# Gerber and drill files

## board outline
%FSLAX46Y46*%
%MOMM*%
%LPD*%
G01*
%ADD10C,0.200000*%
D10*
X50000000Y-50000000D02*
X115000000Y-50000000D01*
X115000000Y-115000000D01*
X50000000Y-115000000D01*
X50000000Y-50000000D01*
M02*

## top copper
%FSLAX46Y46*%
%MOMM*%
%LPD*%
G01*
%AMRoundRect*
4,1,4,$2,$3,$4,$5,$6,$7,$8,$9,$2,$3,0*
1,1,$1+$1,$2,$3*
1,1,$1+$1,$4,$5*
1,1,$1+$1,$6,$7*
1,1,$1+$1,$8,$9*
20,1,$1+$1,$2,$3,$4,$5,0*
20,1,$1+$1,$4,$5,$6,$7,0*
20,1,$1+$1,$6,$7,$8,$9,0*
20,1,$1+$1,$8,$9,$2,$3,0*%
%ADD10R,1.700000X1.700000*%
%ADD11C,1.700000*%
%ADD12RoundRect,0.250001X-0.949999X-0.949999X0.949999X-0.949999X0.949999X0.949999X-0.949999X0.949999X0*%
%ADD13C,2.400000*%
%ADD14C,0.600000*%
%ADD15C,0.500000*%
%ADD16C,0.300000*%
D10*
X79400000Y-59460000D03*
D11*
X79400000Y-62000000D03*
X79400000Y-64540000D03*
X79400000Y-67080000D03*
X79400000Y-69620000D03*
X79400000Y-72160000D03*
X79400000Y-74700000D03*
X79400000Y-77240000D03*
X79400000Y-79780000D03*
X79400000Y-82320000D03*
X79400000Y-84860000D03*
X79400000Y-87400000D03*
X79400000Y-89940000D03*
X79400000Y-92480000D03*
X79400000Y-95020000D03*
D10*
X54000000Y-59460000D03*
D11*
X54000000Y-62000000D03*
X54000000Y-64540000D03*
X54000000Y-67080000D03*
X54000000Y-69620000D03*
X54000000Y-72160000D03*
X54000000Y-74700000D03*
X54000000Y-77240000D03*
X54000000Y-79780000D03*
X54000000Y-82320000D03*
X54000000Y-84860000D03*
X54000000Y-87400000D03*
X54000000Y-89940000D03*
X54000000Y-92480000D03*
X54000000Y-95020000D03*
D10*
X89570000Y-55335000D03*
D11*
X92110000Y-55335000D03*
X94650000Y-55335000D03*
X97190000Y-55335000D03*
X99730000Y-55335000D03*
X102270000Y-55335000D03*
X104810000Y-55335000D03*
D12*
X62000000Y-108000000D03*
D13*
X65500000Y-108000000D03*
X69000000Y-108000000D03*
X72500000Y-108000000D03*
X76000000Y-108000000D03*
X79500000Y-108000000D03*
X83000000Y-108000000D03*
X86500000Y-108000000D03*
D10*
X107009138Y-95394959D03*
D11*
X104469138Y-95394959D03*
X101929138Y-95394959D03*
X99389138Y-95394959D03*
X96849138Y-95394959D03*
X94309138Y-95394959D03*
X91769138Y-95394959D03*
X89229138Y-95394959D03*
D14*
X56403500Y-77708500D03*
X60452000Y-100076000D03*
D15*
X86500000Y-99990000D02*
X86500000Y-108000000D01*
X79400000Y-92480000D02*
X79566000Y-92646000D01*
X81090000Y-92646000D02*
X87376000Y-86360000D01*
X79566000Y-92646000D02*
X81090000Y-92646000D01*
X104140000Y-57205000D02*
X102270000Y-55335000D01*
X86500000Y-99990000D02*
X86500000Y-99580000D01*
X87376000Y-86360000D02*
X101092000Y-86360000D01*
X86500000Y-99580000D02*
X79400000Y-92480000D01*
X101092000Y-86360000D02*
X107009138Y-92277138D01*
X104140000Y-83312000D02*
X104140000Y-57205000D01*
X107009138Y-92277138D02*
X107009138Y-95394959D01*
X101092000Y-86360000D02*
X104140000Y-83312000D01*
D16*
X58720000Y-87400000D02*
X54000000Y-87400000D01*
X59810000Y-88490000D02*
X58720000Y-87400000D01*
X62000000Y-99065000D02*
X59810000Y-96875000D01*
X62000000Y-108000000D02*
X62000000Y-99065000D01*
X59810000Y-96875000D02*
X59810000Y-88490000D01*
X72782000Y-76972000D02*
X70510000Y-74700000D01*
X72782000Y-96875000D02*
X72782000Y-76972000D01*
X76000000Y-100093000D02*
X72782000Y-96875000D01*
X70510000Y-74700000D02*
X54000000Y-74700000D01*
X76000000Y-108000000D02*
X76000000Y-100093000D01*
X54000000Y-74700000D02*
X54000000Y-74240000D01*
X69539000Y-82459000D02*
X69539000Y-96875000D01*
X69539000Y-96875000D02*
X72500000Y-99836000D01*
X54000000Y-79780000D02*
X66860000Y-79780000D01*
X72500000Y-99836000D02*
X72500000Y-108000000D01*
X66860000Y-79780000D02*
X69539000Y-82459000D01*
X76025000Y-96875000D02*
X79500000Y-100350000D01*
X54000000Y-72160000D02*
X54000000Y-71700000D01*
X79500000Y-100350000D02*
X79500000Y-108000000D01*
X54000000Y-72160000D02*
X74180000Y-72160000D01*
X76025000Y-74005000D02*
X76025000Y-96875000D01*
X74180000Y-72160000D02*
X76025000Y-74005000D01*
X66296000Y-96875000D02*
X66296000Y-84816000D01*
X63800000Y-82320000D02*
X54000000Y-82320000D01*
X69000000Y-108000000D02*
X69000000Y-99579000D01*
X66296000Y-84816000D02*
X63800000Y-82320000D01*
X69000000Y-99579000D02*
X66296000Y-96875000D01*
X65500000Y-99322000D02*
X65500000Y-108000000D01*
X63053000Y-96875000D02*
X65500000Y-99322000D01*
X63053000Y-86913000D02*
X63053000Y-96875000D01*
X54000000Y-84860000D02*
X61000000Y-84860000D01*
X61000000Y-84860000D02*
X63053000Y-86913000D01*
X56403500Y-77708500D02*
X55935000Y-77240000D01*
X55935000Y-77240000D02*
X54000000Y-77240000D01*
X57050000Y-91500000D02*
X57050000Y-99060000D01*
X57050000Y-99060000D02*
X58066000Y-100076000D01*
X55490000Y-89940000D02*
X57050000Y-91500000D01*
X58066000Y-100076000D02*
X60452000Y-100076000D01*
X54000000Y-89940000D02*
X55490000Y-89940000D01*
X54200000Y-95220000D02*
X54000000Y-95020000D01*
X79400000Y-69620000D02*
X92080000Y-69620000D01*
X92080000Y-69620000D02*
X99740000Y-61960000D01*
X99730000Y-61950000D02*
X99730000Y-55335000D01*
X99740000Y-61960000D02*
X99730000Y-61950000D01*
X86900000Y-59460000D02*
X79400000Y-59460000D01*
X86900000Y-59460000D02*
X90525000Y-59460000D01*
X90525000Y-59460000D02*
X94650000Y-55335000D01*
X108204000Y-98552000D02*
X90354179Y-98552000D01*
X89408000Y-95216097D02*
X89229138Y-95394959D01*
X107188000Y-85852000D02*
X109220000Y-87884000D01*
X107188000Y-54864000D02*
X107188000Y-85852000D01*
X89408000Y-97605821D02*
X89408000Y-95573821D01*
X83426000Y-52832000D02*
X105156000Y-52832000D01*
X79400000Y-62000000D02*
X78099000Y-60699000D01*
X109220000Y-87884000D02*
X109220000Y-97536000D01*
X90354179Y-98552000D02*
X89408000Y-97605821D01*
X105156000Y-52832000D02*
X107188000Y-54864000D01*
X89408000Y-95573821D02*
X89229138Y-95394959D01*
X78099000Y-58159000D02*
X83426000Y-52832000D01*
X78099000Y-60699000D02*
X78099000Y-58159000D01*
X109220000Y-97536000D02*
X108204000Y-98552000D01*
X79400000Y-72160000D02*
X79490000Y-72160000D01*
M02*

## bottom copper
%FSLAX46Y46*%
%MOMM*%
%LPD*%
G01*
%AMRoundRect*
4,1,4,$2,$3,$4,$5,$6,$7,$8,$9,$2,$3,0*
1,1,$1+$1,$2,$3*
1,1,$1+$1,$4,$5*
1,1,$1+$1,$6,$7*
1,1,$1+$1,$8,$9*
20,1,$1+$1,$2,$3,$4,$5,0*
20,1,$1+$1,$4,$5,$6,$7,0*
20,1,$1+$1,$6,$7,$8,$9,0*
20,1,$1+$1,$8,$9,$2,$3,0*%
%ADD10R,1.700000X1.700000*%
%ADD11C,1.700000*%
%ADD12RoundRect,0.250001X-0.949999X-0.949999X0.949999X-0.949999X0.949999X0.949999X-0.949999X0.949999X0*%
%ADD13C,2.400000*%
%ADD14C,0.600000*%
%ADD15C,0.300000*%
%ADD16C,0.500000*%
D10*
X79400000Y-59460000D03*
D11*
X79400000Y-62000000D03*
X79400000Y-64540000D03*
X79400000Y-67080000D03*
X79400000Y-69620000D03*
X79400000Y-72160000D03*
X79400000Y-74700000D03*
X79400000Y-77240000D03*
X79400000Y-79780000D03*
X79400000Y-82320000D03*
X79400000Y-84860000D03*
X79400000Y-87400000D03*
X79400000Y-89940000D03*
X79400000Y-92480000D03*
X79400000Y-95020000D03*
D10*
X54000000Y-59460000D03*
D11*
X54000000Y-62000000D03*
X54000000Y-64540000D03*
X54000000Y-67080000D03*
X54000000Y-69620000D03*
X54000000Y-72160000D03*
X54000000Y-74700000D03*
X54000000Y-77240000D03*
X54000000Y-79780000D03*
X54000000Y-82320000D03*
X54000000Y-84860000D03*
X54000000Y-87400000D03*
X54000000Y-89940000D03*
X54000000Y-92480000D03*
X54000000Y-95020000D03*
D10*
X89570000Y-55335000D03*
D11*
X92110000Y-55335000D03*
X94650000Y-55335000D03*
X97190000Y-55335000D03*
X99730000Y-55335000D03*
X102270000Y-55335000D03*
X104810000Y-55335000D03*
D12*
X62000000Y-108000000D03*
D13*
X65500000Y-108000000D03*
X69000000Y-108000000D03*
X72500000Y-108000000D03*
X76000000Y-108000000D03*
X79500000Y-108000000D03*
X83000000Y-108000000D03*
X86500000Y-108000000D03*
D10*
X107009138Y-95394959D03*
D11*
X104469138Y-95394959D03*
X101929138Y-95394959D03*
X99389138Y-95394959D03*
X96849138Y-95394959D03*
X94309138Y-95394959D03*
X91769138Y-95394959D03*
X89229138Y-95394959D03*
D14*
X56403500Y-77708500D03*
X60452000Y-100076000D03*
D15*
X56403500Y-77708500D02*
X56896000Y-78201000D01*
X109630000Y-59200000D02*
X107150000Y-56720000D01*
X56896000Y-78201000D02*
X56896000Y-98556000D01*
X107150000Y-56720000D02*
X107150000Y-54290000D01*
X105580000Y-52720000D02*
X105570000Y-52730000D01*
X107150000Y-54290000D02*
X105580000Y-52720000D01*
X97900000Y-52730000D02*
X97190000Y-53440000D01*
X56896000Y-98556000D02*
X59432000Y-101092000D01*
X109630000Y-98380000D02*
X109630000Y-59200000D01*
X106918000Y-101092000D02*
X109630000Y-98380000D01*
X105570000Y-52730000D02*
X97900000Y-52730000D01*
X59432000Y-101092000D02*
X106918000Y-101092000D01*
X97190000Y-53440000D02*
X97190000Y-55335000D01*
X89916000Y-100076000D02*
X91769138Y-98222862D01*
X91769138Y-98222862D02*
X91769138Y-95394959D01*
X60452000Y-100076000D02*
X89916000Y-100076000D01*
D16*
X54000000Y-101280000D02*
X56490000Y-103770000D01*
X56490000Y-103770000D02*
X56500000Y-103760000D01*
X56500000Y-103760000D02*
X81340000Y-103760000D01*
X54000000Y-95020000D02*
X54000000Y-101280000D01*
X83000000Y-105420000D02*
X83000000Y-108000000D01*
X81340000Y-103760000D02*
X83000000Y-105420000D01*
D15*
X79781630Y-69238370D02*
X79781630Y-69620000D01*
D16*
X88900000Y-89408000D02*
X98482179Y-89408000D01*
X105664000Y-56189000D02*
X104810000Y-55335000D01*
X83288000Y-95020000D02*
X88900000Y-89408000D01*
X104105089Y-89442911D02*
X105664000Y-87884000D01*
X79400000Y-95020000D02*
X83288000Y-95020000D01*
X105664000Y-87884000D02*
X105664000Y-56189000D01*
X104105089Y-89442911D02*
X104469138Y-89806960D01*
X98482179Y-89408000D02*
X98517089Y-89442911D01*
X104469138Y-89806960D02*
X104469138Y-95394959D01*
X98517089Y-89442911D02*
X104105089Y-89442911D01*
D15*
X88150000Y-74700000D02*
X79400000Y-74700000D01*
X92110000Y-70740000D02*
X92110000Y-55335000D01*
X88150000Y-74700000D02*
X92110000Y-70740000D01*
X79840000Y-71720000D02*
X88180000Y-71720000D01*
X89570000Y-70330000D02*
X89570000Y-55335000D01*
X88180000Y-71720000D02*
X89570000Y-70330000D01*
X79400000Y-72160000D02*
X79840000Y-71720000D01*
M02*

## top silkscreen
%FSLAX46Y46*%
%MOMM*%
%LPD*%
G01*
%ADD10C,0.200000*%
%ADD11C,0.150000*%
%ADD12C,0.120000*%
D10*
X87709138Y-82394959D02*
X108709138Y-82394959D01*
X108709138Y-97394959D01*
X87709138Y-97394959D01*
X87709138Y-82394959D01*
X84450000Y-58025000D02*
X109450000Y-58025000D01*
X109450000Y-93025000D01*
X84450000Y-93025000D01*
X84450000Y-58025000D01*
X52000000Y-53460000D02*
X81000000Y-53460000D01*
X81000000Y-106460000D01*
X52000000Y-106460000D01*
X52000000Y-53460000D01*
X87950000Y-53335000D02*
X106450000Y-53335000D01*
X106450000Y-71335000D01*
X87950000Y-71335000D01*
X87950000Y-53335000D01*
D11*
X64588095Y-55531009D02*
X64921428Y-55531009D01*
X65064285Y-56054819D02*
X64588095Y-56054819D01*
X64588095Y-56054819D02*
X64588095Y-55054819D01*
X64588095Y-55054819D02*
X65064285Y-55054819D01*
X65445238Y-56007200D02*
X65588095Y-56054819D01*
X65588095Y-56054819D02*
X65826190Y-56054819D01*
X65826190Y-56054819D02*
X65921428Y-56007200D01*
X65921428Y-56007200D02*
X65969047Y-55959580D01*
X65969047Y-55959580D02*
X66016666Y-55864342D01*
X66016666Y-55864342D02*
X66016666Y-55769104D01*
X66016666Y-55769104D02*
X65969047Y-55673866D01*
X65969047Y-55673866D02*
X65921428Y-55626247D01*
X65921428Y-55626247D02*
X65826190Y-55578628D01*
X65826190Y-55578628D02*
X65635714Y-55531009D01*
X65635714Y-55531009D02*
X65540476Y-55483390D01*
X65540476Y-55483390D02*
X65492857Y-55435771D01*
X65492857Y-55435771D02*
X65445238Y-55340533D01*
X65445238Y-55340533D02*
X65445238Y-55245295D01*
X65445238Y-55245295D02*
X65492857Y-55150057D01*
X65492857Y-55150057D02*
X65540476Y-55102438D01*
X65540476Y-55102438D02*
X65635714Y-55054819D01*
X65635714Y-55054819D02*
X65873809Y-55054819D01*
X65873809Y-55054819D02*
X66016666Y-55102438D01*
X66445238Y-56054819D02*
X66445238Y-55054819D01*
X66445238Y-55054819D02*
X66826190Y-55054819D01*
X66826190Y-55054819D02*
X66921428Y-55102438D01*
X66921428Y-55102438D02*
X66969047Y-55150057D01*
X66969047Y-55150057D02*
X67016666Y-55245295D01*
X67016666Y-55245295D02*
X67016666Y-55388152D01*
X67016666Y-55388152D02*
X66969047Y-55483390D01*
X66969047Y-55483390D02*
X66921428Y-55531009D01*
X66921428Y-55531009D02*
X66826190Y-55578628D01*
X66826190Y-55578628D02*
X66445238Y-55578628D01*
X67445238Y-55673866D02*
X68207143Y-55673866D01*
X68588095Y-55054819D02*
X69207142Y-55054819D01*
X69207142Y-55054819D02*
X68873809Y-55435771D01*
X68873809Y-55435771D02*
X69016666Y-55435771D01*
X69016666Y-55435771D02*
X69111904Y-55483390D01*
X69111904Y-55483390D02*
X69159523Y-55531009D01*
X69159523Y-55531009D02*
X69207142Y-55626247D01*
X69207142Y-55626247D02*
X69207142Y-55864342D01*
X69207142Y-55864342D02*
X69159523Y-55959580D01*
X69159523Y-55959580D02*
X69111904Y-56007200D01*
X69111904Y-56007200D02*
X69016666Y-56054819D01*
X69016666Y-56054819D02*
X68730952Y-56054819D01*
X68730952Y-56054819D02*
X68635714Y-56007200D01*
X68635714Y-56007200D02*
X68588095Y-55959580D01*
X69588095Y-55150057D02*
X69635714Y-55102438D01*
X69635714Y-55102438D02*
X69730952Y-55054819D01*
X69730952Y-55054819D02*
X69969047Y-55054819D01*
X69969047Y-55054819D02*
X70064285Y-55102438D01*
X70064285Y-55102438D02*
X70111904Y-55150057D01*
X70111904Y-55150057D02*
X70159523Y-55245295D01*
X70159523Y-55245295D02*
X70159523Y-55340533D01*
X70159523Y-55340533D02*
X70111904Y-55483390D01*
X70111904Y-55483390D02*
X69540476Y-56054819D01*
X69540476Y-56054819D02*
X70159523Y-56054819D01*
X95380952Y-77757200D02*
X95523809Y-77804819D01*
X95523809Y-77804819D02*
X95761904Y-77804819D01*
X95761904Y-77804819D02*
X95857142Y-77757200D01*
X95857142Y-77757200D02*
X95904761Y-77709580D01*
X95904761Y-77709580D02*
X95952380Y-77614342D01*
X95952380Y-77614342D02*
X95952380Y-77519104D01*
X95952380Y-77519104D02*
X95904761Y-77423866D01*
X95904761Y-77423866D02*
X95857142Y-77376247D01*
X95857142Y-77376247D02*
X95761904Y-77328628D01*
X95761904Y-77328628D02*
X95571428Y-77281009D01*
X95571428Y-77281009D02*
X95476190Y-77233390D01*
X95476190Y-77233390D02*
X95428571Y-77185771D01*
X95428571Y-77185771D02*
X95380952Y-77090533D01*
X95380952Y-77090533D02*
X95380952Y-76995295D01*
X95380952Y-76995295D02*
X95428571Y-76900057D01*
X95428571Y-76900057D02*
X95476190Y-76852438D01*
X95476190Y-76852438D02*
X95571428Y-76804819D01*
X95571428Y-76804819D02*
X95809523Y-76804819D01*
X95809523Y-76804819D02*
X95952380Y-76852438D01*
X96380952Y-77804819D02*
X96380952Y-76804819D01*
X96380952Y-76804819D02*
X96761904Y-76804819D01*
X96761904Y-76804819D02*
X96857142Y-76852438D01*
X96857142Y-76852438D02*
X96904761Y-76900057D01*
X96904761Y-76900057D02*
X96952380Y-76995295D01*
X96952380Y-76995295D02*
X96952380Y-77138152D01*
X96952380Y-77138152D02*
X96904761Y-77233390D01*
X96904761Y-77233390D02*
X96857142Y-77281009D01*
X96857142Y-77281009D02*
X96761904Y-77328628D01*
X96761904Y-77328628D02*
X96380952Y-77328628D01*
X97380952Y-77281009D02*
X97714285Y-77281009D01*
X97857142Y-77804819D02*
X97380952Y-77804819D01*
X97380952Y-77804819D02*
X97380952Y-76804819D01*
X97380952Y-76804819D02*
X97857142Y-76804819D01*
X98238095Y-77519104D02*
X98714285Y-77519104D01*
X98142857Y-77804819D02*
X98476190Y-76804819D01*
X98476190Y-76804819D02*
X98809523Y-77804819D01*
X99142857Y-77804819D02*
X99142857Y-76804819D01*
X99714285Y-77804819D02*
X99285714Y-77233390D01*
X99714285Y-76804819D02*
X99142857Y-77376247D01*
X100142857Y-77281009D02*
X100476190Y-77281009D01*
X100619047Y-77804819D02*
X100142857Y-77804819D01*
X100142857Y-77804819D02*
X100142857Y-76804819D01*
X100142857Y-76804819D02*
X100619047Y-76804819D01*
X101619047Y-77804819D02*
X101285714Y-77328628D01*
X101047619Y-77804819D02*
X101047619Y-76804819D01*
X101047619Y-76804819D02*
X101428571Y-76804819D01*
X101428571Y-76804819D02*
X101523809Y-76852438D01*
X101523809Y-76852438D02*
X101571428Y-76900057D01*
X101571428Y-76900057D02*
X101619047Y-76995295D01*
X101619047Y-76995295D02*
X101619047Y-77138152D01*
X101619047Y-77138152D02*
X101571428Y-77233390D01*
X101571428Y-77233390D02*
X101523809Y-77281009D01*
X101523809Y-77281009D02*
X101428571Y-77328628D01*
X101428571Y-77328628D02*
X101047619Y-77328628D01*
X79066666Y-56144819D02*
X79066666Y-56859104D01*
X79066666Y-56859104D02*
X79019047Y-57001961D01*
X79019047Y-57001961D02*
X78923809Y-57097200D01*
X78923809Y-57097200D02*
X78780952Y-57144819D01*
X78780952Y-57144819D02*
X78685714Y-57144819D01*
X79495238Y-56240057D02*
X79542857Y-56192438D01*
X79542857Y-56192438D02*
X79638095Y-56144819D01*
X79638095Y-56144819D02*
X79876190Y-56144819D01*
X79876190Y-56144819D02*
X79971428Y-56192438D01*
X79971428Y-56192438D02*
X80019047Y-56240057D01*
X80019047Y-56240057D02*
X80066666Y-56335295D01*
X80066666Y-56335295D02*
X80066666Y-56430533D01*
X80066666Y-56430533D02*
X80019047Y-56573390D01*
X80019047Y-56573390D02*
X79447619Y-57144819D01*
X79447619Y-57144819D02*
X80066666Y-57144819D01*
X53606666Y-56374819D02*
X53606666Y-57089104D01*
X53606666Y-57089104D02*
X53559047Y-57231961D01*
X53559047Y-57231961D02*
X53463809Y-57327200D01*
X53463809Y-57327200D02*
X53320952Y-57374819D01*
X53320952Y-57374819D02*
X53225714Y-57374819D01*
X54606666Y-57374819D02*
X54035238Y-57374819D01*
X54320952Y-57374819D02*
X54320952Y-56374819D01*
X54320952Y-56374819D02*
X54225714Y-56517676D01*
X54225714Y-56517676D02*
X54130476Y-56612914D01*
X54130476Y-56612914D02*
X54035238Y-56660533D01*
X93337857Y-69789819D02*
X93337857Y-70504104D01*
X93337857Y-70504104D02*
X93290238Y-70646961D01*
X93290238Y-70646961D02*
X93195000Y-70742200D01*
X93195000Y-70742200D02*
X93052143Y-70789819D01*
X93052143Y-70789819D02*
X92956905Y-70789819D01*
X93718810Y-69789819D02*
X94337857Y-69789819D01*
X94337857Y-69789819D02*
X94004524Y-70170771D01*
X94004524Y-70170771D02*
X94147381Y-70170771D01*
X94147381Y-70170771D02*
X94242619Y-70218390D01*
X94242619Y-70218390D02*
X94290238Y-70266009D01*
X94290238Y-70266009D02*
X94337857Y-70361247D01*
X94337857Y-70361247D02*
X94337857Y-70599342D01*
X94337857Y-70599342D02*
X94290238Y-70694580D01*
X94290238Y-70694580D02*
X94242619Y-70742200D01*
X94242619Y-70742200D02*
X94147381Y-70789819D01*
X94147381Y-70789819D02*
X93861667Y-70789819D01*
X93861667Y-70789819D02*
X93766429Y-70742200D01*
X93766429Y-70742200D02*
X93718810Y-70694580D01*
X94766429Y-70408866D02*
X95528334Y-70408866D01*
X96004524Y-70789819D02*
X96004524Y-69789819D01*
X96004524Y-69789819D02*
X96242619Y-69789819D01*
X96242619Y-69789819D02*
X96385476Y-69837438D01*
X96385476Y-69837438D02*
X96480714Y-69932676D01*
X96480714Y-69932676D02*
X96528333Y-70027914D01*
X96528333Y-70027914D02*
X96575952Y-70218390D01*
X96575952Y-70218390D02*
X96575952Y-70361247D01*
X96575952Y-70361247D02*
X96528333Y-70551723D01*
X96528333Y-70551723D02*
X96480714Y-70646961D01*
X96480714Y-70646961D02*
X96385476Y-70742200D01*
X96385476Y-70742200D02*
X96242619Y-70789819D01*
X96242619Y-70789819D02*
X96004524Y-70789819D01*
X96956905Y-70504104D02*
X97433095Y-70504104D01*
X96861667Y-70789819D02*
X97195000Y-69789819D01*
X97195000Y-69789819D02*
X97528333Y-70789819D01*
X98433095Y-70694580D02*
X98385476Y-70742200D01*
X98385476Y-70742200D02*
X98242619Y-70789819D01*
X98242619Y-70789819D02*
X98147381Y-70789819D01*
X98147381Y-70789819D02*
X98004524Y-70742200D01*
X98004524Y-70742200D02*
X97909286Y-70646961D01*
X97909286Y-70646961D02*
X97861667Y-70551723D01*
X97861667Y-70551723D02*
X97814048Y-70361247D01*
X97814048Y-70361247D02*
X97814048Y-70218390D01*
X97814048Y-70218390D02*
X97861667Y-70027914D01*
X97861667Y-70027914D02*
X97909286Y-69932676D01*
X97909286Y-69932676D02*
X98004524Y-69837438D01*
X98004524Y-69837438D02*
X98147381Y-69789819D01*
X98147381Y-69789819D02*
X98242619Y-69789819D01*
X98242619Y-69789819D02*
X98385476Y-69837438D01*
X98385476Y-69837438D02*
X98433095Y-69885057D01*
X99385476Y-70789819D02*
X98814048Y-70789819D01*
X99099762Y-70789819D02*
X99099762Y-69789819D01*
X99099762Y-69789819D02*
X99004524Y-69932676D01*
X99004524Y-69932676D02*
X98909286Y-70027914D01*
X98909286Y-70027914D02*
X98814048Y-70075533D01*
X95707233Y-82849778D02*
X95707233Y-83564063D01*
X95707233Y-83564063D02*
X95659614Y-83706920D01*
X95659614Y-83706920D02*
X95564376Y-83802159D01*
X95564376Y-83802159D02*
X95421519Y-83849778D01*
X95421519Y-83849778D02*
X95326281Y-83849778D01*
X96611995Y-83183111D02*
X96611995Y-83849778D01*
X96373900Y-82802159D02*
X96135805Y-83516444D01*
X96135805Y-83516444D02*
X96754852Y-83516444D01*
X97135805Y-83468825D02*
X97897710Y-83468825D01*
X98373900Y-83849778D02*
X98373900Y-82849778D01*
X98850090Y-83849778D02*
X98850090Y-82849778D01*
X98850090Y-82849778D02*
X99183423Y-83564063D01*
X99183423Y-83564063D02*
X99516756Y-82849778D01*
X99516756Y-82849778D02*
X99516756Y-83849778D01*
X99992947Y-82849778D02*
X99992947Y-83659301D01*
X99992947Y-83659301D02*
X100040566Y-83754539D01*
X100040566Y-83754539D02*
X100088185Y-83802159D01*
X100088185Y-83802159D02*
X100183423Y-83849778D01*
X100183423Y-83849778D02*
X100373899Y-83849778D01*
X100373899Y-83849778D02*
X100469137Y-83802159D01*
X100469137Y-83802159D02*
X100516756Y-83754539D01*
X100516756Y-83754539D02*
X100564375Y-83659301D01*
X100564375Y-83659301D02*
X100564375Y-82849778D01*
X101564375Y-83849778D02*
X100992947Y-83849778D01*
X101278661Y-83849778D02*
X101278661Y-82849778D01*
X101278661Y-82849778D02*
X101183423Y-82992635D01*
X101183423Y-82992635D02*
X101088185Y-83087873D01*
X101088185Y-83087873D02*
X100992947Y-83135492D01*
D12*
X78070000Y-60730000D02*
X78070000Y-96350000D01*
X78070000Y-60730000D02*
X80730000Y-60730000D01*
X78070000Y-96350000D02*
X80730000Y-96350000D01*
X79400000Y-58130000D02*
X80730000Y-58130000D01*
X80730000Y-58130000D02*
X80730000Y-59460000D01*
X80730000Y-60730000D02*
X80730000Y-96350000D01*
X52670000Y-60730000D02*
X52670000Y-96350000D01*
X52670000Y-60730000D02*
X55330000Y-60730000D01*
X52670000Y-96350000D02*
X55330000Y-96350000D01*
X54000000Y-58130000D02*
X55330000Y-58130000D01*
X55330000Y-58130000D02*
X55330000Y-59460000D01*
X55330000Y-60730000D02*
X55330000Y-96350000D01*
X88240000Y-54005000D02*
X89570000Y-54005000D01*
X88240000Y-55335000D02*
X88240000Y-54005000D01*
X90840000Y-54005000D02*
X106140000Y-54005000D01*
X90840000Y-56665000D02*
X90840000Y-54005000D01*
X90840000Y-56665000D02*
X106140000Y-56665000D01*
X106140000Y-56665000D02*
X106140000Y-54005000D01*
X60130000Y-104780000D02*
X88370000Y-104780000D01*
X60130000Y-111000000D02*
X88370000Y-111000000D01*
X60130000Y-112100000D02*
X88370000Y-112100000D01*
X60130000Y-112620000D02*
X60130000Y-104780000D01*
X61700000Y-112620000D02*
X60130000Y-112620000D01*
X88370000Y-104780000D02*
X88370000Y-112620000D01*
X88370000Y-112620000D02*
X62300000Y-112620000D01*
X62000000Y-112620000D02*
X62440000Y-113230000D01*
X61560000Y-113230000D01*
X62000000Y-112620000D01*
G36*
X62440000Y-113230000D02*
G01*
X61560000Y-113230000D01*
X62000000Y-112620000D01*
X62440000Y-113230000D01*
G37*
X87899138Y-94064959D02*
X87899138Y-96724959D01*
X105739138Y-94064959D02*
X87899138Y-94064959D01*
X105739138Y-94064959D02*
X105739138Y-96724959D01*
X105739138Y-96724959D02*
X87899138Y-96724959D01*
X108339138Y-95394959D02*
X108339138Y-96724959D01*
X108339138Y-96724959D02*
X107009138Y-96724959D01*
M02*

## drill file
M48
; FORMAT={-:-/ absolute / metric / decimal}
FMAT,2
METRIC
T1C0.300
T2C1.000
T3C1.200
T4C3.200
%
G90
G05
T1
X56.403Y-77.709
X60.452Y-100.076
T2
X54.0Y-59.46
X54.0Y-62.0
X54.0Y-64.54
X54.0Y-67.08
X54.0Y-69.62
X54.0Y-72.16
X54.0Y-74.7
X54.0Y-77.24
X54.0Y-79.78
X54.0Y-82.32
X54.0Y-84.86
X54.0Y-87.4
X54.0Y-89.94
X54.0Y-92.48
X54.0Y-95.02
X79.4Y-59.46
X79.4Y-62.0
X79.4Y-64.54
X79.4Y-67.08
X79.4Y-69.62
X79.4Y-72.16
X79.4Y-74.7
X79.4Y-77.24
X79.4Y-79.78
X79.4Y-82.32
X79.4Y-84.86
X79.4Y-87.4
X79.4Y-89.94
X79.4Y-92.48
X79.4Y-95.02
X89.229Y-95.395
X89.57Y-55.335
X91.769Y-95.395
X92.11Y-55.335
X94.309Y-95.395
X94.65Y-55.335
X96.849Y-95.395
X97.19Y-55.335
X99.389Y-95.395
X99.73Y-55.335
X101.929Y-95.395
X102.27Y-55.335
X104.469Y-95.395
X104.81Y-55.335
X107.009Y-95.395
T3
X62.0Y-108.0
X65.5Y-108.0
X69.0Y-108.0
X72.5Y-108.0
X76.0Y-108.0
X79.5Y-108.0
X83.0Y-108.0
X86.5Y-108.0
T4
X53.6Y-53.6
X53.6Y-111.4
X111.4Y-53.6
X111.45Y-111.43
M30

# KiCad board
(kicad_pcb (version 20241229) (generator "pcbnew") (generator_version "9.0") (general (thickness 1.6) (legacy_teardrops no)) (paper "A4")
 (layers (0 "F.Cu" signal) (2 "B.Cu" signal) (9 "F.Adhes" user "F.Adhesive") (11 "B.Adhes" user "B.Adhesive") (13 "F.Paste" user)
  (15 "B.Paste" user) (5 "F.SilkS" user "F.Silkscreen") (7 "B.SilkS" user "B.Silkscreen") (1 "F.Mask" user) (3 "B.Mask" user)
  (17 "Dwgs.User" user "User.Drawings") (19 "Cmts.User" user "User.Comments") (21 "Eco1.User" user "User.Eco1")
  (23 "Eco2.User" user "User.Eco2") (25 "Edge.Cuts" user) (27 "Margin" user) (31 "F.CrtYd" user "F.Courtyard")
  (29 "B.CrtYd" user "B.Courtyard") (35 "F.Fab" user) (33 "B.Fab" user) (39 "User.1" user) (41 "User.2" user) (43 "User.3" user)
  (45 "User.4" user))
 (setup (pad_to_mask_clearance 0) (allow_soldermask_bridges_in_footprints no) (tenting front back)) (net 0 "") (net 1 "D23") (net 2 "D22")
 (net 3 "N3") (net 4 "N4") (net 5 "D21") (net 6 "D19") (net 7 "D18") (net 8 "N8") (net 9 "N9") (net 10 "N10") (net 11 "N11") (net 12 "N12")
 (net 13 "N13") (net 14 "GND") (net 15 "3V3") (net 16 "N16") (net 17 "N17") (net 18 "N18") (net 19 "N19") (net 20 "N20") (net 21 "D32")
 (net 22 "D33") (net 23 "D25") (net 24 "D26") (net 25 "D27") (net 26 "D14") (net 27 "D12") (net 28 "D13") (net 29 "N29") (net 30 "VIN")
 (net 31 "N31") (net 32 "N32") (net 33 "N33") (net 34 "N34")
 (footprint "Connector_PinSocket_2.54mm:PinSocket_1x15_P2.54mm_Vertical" (layer "F.Cu") (at 79.4 59.46)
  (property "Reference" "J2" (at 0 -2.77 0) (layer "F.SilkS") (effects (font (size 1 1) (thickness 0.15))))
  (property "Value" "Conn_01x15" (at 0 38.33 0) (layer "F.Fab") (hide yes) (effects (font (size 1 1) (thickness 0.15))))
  (fp_line (start -1.33 1.27) (end -1.33 36.89) (stroke (width 0.12) (type solid)) (layer "F.SilkS"))
  (fp_line (start -1.33 1.27) (end 1.33 1.27) (stroke (width 0.12) (type solid)) (layer "F.SilkS"))
  (fp_line (start -1.33 36.89) (end 1.33 36.89) (stroke (width 0.12) (type solid)) (layer "F.SilkS"))
  (fp_line (start 0 -1.33) (end 1.33 -1.33) (stroke (width 0.12) (type solid)) (layer "F.SilkS"))
  (fp_line (start 1.33 -1.33) (end 1.33 0) (stroke (width 0.12) (type solid)) (layer "F.SilkS"))
  (fp_line (start 1.33 1.27) (end 1.33 36.89) (stroke (width 0.12) (type solid)) (layer "F.SilkS"))
  (pad "1" thru_hole rect (at 0 0) (size 1.7 1.7) (drill 1) (layers "*.Cu" "*.Mask") (remove_unused_layers no) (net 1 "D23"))
  (pad "2" thru_hole circle (at 0 2.54) (size 1.7 1.7) (drill 1) (layers "*.Cu" "*.Mask") (remove_unused_layers no) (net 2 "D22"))
  (pad "3" thru_hole circle (at 0 5.08) (size 1.7 1.7) (drill 1) (layers "*.Cu" "*.Mask") (remove_unused_layers no) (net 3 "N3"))
  (pad "4" thru_hole circle (at 0 7.62) (size 1.7 1.7) (drill 1) (layers "*.Cu" "*.Mask") (remove_unused_layers no) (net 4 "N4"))
  (pad "5" thru_hole circle (at 0 10.16) (size 1.7 1.7) (drill 1) (layers "*.Cu" "*.Mask") (remove_unused_layers no) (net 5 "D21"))
  (pad "6" thru_hole circle (at 0 12.7) (size 1.7 1.7) (drill 1) (layers "*.Cu" "*.Mask") (remove_unused_layers no) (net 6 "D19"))
  (pad "7" thru_hole circle (at 0 15.24) (size 1.7 1.7) (drill 1) (layers "*.Cu" "*.Mask") (remove_unused_layers no) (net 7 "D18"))
  (pad "8" thru_hole circle (at 0 17.78) (size 1.7 1.7) (drill 1) (layers "*.Cu" "*.Mask") (remove_unused_layers no) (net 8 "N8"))
  (pad "9" thru_hole circle (at 0 20.32) (size 1.7 1.7) (drill 1) (layers "*.Cu" "*.Mask") (remove_unused_layers no) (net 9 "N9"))
  (pad "10" thru_hole circle (at 0 22.86) (size 1.7 1.7) (drill 1) (layers "*.Cu" "*.Mask") (remove_unused_layers no) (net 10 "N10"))
  (pad "11" thru_hole circle (at 0 25.4) (size 1.7 1.7) (drill 1) (layers "*.Cu" "*.Mask") (remove_unused_layers no) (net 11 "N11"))
  (pad "12" thru_hole circle (at 0 27.94) (size 1.7 1.7) (drill 1) (layers "*.Cu" "*.Mask") (remove_unused_layers no) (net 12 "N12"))
  (pad "13" thru_hole circle (at 0 30.48) (size 1.7 1.7) (drill 1) (layers "*.Cu" "*.Mask") (remove_unused_layers no) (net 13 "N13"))
  (pad "14" thru_hole circle (at 0 33.02) (size 1.7 1.7) (drill 1) (layers "*.Cu" "*.Mask") (remove_unused_layers no) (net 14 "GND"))
  (pad "15" thru_hole circle (at 0 35.56) (size 1.7 1.7) (drill 1) (layers "*.Cu" "*.Mask") (remove_unused_layers no) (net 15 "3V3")))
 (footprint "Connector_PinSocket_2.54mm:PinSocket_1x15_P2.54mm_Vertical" (layer "F.Cu") (at 54 59.46)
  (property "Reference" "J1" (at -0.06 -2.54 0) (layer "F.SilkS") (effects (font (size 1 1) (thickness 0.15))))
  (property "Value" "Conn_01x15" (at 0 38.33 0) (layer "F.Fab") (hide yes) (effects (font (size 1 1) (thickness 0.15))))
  (fp_line (start -1.33 1.27) (end -1.33 36.89) (stroke (width 0.12) (type solid)) (layer "F.SilkS"))
  (fp_line (start -1.33 1.27) (end 1.33 1.27) (stroke (width 0.12) (type solid)) (layer "F.SilkS"))
  (fp_line (start -1.33 36.89) (end 1.33 36.89) (stroke (width 0.12) (type solid)) (layer "F.SilkS"))
  (fp_line (start 0 -1.33) (end 1.33 -1.33) (stroke (width 0.12) (type solid)) (layer "F.SilkS"))
  (fp_line (start 1.33 -1.33) (end 1.33 0) (stroke (width 0.12) (type solid)) (layer "F.SilkS"))
  (fp_line (start 1.33 1.27) (end 1.33 36.89) (stroke (width 0.12) (type solid)) (layer "F.SilkS"))
  (pad "1" thru_hole rect (at 0 0) (size 1.7 1.7) (drill 1) (layers "*.Cu" "*.Mask") (remove_unused_layers no) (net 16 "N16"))
  (pad "2" thru_hole circle (at 0 2.54) (size 1.7 1.7) (drill 1) (layers "*.Cu" "*.Mask") (remove_unused_layers no) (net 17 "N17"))
  (pad "3" thru_hole circle (at 0 5.08) (size 1.7 1.7) (drill 1) (layers "*.Cu" "*.Mask") (remove_unused_layers no) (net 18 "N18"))
  (pad "4" thru_hole circle (at 0 7.62) (size 1.7 1.7) (drill 1) (layers "*.Cu" "*.Mask") (remove_unused_layers no) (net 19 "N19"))
  (pad "5" thru_hole circle (at 0 10.16) (size 1.7 1.7) (drill 1) (layers "*.Cu" "*.Mask") (remove_unused_layers no) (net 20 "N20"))
  (pad "6" thru_hole circle (at 0 12.7) (size 1.7 1.7) (drill 1) (layers "*.Cu" "*.Mask") (remove_unused_layers no) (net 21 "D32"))
  (pad "7" thru_hole circle (at 0 15.24) (size 1.7 1.7) (drill 1) (layers "*.Cu" "*.Mask") (remove_unused_layers no) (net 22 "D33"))
  (pad "8" thru_hole circle (at 0 17.78) (size 1.7 1.7) (drill 1) (layers "*.Cu" "*.Mask") (remove_unused_layers no) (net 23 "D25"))
  (pad "9" thru_hole circle (at 0 20.32) (size 1.7 1.7) (drill 1) (layers "*.Cu" "*.Mask") (remove_unused_layers no) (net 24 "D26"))
  (pad "10" thru_hole circle (at 0 22.86) (size 1.7 1.7) (drill 1) (layers "*.Cu" "*.Mask") (remove_unused_layers no) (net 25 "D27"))
  (pad "11" thru_hole circle (at 0 25.4) (size 1.7 1.7) (drill 1) (layers "*.Cu" "*.Mask") (remove_unused_layers no) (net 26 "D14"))
  (pad "12" thru_hole circle (at 0 27.94) (size 1.7 1.7) (drill 1) (layers "*.Cu" "*.Mask") (remove_unused_layers no) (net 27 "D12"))
  (pad "13" thru_hole circle (at 0 30.48) (size 1.7 1.7) (drill 1) (layers "*.Cu" "*.Mask") (remove_unused_layers no) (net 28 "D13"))
  (pad "14" thru_hole circle (at 0 33.02) (size 1.7 1.7) (drill 1) (layers "*.Cu" "*.Mask") (remove_unused_layers no) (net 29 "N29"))
  (pad "15" thru_hole circle (at 0 35.56) (size 1.7 1.7) (drill 1) (layers "*.Cu" "*.Mask") (remove_unused_layers no) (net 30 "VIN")))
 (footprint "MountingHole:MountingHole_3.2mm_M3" (layer "F.Cu") (at 53.6 53.6)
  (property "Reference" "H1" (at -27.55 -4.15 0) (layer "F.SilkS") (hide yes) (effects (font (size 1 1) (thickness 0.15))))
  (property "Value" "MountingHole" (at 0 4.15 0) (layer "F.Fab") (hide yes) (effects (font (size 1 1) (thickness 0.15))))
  (pad "" np_thru_hole circle (at 0 0) (size 3.2 3.2) (drill 3.2) (layers "*.Cu" "*.Mask")))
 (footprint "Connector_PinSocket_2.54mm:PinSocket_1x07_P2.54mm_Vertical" (layer "F.Cu") (at 89.57 55.335 90)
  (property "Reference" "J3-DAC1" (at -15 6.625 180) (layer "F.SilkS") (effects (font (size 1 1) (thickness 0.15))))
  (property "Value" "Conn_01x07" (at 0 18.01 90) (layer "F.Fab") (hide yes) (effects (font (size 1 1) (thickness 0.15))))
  (fp_line (start 1.33 -1.33) (end 1.33 0) (stroke (width 0.12) (type solid)) (layer "F.SilkS"))
  (fp_line (start 0 -1.33) (end 1.33 -1.33) (stroke (width 0.12) (type solid)) (layer "F.SilkS"))
  (fp_line (start 1.33 1.27) (end 1.33 16.57) (stroke (width 0.12) (type solid)) (layer "F.SilkS"))
  (fp_line (start -1.33 1.27) (end 1.33 1.27) (stroke (width 0.12) (type solid)) (layer "F.SilkS"))
  (fp_line (start -1.33 1.27) (end -1.33 16.57) (stroke (width 0.12) (type solid)) (layer "F.SilkS"))
  (fp_line (start -1.33 16.57) (end 1.33 16.57) (stroke (width 0.12) (type solid)) (layer "F.SilkS"))
  (pad "1" thru_hole rect (at 0 0 90) (size 1.7 1.7) (drill 1) (layers "*.Cu" "*.Mask") (remove_unused_layers no) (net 6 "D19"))
  (pad "2" thru_hole circle (at 0 2.54 90) (size 1.7 1.7) (drill 1) (layers "*.Cu" "*.Mask") (remove_unused_layers no) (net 7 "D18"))
  (pad "3" thru_hole circle (at 0 5.08 90) (size 1.7 1.7) (drill 1) (layers "*.Cu" "*.Mask") (remove_unused_layers no) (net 1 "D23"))
  (pad "4" thru_hole circle (at 0 7.62 90) (size 1.7 1.7) (drill 1) (layers "*.Cu" "*.Mask") (remove_unused_layers no) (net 23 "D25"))
  (pad "5" thru_hole circle (at 0 10.16 90) (size 1.7 1.7) (drill 1) (layers "*.Cu" "*.Mask") (remove_unused_layers no) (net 5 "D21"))
  (pad "6" thru_hole circle (at 0 12.7 90) (size 1.7 1.7) (drill 1) (layers "*.Cu" "*.Mask") (remove_unused_layers no) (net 14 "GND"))
  (pad "7" thru_hole circle (at 0 15.24 90) (size 1.7 1.7) (drill 1) (layers "*.Cu" "*.Mask") (remove_unused_layers no) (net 15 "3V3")))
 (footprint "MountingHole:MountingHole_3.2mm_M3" (layer "F.Cu") (at 53.6 111.4)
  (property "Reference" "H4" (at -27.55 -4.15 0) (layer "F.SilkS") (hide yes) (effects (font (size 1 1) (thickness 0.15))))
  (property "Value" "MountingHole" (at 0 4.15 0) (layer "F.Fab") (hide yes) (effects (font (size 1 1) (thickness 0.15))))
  (pad "" np_thru_hole circle (at 0 0) (size 3.2 3.2) (drill 3.2) (layers "*.Cu" "*.Mask")))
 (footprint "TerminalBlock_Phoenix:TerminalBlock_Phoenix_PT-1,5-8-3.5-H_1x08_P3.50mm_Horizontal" (layer "F.Cu") (at 62 108)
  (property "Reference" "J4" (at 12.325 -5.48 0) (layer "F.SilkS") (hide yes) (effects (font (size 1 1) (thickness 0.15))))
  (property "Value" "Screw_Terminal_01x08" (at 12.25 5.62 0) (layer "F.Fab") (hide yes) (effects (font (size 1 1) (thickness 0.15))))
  (fp_line (start -1.87 -3.22) (end 26.37 -3.22) (stroke (width 0.12) (type solid)) (layer "F.SilkS"))
  (fp_line (start -1.87 3) (end 26.37 3) (stroke (width 0.12) (type solid)) (layer "F.SilkS"))
  (fp_line (start -1.87 4.1) (end 26.37 4.1) (stroke (width 0.12) (type solid)) (layer "F.SilkS"))
  (fp_line (start -1.87 4.62) (end -1.87 -3.22) (stroke (width 0.12) (type solid)) (layer "F.SilkS"))
  (fp_line (start -0.3 4.62) (end -1.87 4.62) (stroke (width 0.12) (type solid)) (layer "F.SilkS"))
  (fp_line (start 26.37 -3.22) (end 26.37 4.62) (stroke (width 0.12) (type solid)) (layer "F.SilkS"))
  (fp_line (start 26.37 4.62) (end 0.3 4.62) (stroke (width 0.12) (type solid)) (layer "F.SilkS"))
  (fp_poly (pts (xy 0 4.62) (xy 0.44 5.23) (xy -0.44 5.23)) (stroke (width 0.12) (type solid)) (fill yes) (layer "F.SilkS"))
  (pad "1" thru_hole roundrect (at 0 0) (size 2.4 2.4) (drill 1.2) (layers "*.Cu" "*.Mask") (remove_unused_layers no)
   (roundrect_rratio 0.104167) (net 27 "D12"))
  (pad "2" thru_hole circle (at 3.5 0) (size 2.4 2.4) (drill 1.2) (layers "*.Cu" "*.Mask") (remove_unused_layers no) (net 26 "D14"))
  (pad "3" thru_hole circle (at 7 0) (size 2.4 2.4) (drill 1.2) (layers "*.Cu" "*.Mask") (remove_unused_layers no) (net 25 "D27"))
  (pad "4" thru_hole circle (at 10.5 0) (size 2.4 2.4) (drill 1.2) (layers "*.Cu" "*.Mask") (remove_unused_layers no) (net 24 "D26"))
  (pad "5" thru_hole circle (at 14 0) (size 2.4 2.4) (drill 1.2) (layers "*.Cu" "*.Mask") (remove_unused_layers no) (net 22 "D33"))
  (pad "6" thru_hole circle (at 17.5 0) (size 2.4 2.4) (drill 1.2) (layers "*.Cu" "*.Mask") (remove_unused_layers no) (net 21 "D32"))
  (pad "7" thru_hole circle (at 21 0) (size 2.4 2.4) (drill 1.2) (layers "*.Cu" "*.Mask") (remove_unused_layers no) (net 30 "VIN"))
  (pad "8" thru_hole circle (at 24.5 0) (size 2.4 2.4) (drill 1.2) (layers "*.Cu" "*.Mask") (remove_unused_layers no) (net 14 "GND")))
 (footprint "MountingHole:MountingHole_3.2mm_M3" (layer "F.Cu") (at 111.45 111.43)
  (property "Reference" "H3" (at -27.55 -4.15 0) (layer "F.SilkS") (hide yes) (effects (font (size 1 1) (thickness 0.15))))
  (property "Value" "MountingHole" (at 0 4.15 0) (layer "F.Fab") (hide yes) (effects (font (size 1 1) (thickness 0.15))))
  (pad "" np_thru_hole circle (at 0 0) (size 3.2 3.2) (drill 3.2) (layers "*.Cu" "*.Mask")))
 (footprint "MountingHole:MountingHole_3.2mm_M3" (layer "F.Cu") (at 111.4 53.6)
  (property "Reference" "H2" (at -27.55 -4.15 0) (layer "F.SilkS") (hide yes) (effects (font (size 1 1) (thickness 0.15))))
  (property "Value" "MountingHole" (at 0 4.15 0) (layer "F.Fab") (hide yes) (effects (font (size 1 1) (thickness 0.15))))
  (pad "" np_thru_hole circle (at 0 0) (size 3.2 3.2) (drill 3.2) (layers "*.Cu" "*.Mask")))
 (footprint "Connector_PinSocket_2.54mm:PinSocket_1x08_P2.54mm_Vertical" (layer "F.Cu") (at 107.009138 95.394959 -90)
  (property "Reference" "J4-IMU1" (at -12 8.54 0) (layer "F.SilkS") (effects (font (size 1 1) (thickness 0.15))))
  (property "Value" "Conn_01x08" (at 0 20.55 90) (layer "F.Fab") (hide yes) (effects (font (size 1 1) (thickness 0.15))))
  (fp_line (start -1.33 19.11) (end 1.33 19.11) (stroke (width 0.12) (type solid)) (layer "F.SilkS"))
  (fp_line (start -1.33 1.27) (end -1.33 19.11) (stroke (width 0.12) (type solid)) (layer "F.SilkS"))
  (fp_line (start -1.33 1.27) (end 1.33 1.27) (stroke (width 0.12) (type solid)) (layer "F.SilkS"))
  (fp_line (start 1.33 1.27) (end 1.33 19.11) (stroke (width 0.12) (type solid)) (layer "F.SilkS"))
  (fp_line (start 0 -1.33) (end 1.33 -1.33) (stroke (width 0.12) (type solid)) (layer "F.SilkS"))
  (fp_line (start 1.33 -1.33) (end 1.33 0) (stroke (width 0.12) (type solid)) (layer "F.SilkS"))
  (pad "1" thru_hole rect (at 0 0 270) (size 1.7 1.7) (drill 1) (layers "*.Cu" "*.Mask") (remove_unused_layers no) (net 14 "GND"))
  (pad "2" thru_hole circle (at 0 2.54 270) (size 1.7 1.7) (drill 1) (layers "*.Cu" "*.Mask") (remove_unused_layers no) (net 15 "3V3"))
  (pad "3" thru_hole circle (at 0 5.08 270) (size 1.7 1.7) (drill 1) (layers "*.Cu" "*.Mask") (remove_unused_layers no) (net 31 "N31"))
  (pad "4" thru_hole circle (at 0 7.62 270) (size 1.7 1.7) (drill 1) (layers "*.Cu" "*.Mask") (remove_unused_layers no) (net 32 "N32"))
  (pad "5" thru_hole circle (at 0 10.16 270) (size 1.7 1.7) (drill 1) (layers "*.Cu" "*.Mask") (remove_unused_layers no) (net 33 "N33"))
  (pad "6" thru_hole circle (at 0 12.7 270) (size 1.7 1.7) (drill 1) (layers "*.Cu" "*.Mask") (remove_unused_layers no) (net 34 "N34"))
  (pad "7" thru_hole circle (at 0 15.24 270) (size 1.7 1.7) (drill 1) (layers "*.Cu" "*.Mask") (remove_unused_layers no) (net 28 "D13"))
  (pad "8" thru_hole circle (at 0 17.78 270) (size 1.7 1.7) (drill 1) (layers "*.Cu" "*.Mask") (remove_unused_layers no) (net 2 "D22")))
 (gr_rect (start 87.709138 82.394959) (end 108.709138 97.394959) (stroke (width 0.2) (type solid)) (fill no) (layer "F.SilkS"))
 (gr_rect (start 84.45 58.025) (end 109.45 93.025) (stroke (width 0.2) (type solid)) (fill no) (layer "F.SilkS"))
 (gr_rect (start 52 53.46) (end 81 106.46) (stroke (width 0.2) (type solid)) (fill no) (layer "F.SilkS"))
 (gr_rect (start 87.95 53.335) (end 106.45 71.335) (stroke (width 0.2) (type solid)) (fill no) (layer "F.SilkS"))
 (gr_rect (start 50 50) (end 115 115) (stroke (width 0.2) (type solid)) (fill no) (layer "Edge.Cuts"))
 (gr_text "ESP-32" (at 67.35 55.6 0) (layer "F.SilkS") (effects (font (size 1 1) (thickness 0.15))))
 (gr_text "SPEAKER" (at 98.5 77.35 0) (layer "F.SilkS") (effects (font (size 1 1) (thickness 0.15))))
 (segment (start 86.5 99.99) (end 86.5 108) (width 0.5) (layer "F.Cu") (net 14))
 (segment (start 79.4 92.48) (end 79.566 92.646) (width 0.5) (layer "F.Cu") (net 14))
 (segment (start 81.09 92.646) (end 87.376 86.36) (width 0.5) (layer "F.Cu") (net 14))
 (segment (start 79.566 92.646) (end 81.09 92.646) (width 0.5) (layer "F.Cu") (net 14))
 (segment (start 104.14 57.205) (end 102.27 55.335) (width 0.5) (layer "F.Cu") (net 14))
 (segment (start 86.5 99.99) (end 86.5 99.58) (width 0.5) (layer "F.Cu") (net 14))
 (segment (start 87.376 86.36) (end 101.092 86.36) (width 0.5) (layer "F.Cu") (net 14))
 (segment (start 86.5 99.58) (end 79.4 92.48) (width 0.5) (layer "F.Cu") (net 14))
 (segment (start 101.092 86.36) (end 107.009138 92.277138) (width 0.5) (layer "F.Cu") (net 14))
 (segment (start 104.14 83.312) (end 104.14 57.205) (width 0.5) (layer "F.Cu") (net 14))
 (segment (start 107.009138 92.277138) (end 107.009138 95.394959) (width 0.5) (layer "F.Cu") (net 14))
 (segment (start 101.092 86.36) (end 104.14 83.312) (width 0.5) (layer "F.Cu") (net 14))
 (segment (start 58.72 87.4) (end 54 87.4) (width 0.3) (layer "F.Cu") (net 27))
 (segment (start 59.81 88.49) (end 58.72 87.4) (width 0.3) (layer "F.Cu") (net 27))
 (segment (start 62 99.065) (end 59.81 96.875) (width 0.3) (layer "F.Cu") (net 27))
 (segment (start 62 108) (end 62 99.065) (width 0.3) (layer "F.Cu") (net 27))
 (segment (start 59.81 96.875) (end 59.81 88.49) (width 0.3) (layer "F.Cu") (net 27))
 (segment (start 72.782 76.972) (end 70.51 74.7) (width 0.3) (layer "F.Cu") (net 22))
 (segment (start 72.782 96.875) (end 72.782 76.972) (width 0.3) (layer "F.Cu") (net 22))
 (segment (start 76 100.093) (end 72.782 96.875) (width 0.3) (layer "F.Cu") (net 22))
 (segment (start 70.51 74.7) (end 54 74.7) (width 0.3) (layer "F.Cu") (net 22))
 (segment (start 76 108) (end 76 100.093) (width 0.3) (layer "F.Cu") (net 22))
 (segment (start 54 74.7) (end 54 74.24) (width 0.3) (layer "F.Cu") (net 22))
 (segment (start 69.539 82.459) (end 69.539 96.875) (width 0.3) (layer "F.Cu") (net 24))
 (segment (start 69.539 96.875) (end 72.5 99.836) (width 0.3) (layer "F.Cu") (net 24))
 (segment (start 54 79.78) (end 66.86 79.78) (width 0.3) (layer "F.Cu") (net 24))
 (segment (start 72.5 99.836) (end 72.5 108) (width 0.3) (layer "F.Cu") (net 24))
 (segment (start 66.86 79.78) (end 69.539 82.459) (width 0.3) (layer "F.Cu") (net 24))
 (segment (start 76.025 96.875) (end 79.5 100.35) (width 0.3) (layer "F.Cu") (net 21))
 (segment (start 54 72.16) (end 54 71.7) (width 0.3) (layer "F.Cu") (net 21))
 (segment (start 79.5 100.35) (end 79.5 108) (width 0.3) (layer "F.Cu") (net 21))
 (segment (start 54 72.16) (end 74.18 72.16) (width 0.3) (layer "F.Cu") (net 21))
 (segment (start 76.025 74.005) (end 76.025 96.875) (width 0.3) (layer "F.Cu") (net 21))
 (segment (start 74.18 72.16) (end 76.025 74.005) (width 0.3) (layer "F.Cu") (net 21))
 (segment (start 66.296 96.875) (end 66.296 84.816) (width 0.3) (layer "F.Cu") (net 25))
 (segment (start 63.8 82.32) (end 54 82.32) (width 0.3) (layer "F.Cu") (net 25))
 (segment (start 69 108) (end 69 99.579) (width 0.3) (layer "F.Cu") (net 25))
 (segment (start 66.296 84.816) (end 63.8 82.32) (width 0.3) (layer "F.Cu") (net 25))
 (segment (start 69 99.579) (end 66.296 96.875) (width 0.3) (layer "F.Cu") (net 25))
 (segment (start 65.5 99.322) (end 65.5 108) (width 0.3) (layer "F.Cu") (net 26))
 (segment (start 63.053 96.875) (end 65.5 99.322) (width 0.3) (layer "F.Cu") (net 26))
 (segment (start 63.053 86.913) (end 63.053 96.875) (width 0.3) (layer "F.Cu") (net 26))
 (segment (start 54 84.86) (end 61 84.86) (width 0.3) (layer "F.Cu") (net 26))
 (segment (start 61 84.86) (end 63.053 86.913) (width 0.3) (layer "F.Cu") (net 26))
 (segment (start 56.4035 77.7085) (end 55.935 77.24) (width 0.3) (layer "F.Cu") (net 23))
 (segment (start 55.935 77.24) (end 54 77.24) (width 0.3) (layer "F.Cu") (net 23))
 (via (at 56.4035 77.7085) (size 0.6) (drill 0.3) (layers "F.Cu" "B.Cu") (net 23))
 (segment (start 56.4035 77.7085) (end 56.896 78.201) (width 0.3) (layer "B.Cu") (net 23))
 (segment (start 109.63 59.2) (end 107.15 56.72) (width 0.3) (layer "B.Cu") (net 23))
 (segment (start 56.896 78.201) (end 56.896 98.556) (width 0.3) (layer "B.Cu") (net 23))
 (segment (start 107.15 56.72) (end 107.15 54.29) (width 0.3) (layer "B.Cu") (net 23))
 (segment (start 105.58 52.72) (end 105.57 52.73) (width 0.3) (layer "B.Cu") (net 23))
 (segment (start 107.15 54.29) (end 105.58 52.72) (width 0.3) (layer "B.Cu") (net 23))
 (segment (start 97.9 52.73) (end 97.19 53.44) (width 0.3) (layer "B.Cu") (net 23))
 (segment (start 56.896 98.556) (end 59.432 101.092) (width 0.3) (layer "B.Cu") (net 23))
 (segment (start 109.63 98.38) (end 109.63 59.2) (width 0.3) (layer "B.Cu") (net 23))
 (segment (start 106.918 101.092) (end 109.63 98.38) (width 0.3) (layer "B.Cu") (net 23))
 (segment (start 105.57 52.73) (end 97.9 52.73) (width 0.3) (layer "B.Cu") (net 23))
 (segment (start 59.432 101.092) (end 106.918 101.092) (width 0.3) (layer "B.Cu") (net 23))
 (segment (start 97.19 53.44) (end 97.19 55.335) (width 0.3) (layer "B.Cu") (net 23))
 (segment (start 57.05 91.5) (end 57.05 99.06) (width 0.3) (layer "F.Cu") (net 28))
 (segment (start 57.05 99.06) (end 58.066 100.076) (width 0.3) (layer "F.Cu") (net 28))
 (segment (start 55.49 89.94) (end 57.05 91.5) (width 0.3) (layer "F.Cu") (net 28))
 (segment (start 58.066 100.076) (end 60.452 100.076) (width 0.3) (layer "F.Cu") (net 28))
 (segment (start 54 89.94) (end 55.49 89.94) (width 0.3) (layer "F.Cu") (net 28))
 (via (at 60.452 100.076) (size 0.6) (drill 0.3) (layers "F.Cu" "B.Cu") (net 28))
 (segment (start 89.916 100.076) (end 91.769138 98.222862) (width 0.3) (layer "B.Cu") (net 28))
 (segment (start 91.769138 98.222862) (end 91.769138 95.394959) (width 0.3) (layer "B.Cu") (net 28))
 (segment (start 60.452 100.076) (end 89.916 100.076) (width 0.3) (layer "B.Cu") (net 28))
 (segment (start 54.2 95.22) (end 54 95.02) (width 0.3) (layer "F.Cu") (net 30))
 (segment (start 54 101.28) (end 56.49 103.77) (width 0.5) (layer "B.Cu") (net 30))
 (segment (start 56.49 103.77) (end 56.5 103.76) (width 0.5) (layer "B.Cu") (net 30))
 (segment (start 56.5 103.76) (end 81.34 103.76) (width 0.5) (layer "B.Cu") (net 30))
 (segment (start 54 95.02) (end 54 101.28) (width 0.5) (layer "B.Cu") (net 30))
 (segment (start 83 105.42) (end 83 108) (width 0.5) (layer "B.Cu") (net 30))
 (segment (start 81.34 103.76) (end 83 105.42) (width 0.5) (layer "B.Cu") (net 30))
 (segment (start 79.4 69.62) (end 92.08 69.62) (width 0.3) (layer "F.Cu") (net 5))
 (segment (start 92.08 69.62) (end 99.74 61.96) (width 0.3) (layer "F.Cu") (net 5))
 (segment (start 99.73 61.95) (end 99.73 55.335) (width 0.3) (layer "F.Cu") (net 5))
 (segment (start 99.74 61.96) (end 99.73 61.95) (width 0.3) (layer "F.Cu") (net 5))
 (segment (start 79.78163 69.23837) (end 79.78163 69.62) (width 0.3) (layer "B.Cu") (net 5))
 (segment (start 86.9 59.46) (end 79.4 59.46) (width 0.3) (layer "F.Cu") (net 1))
 (segment (start 86.9 59.46) (end 90.525 59.46) (width 0.3) (layer "F.Cu") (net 1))
 (segment (start 90.525 59.46) (end 94.65 55.335) (width 0.3) (layer "F.Cu") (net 1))
 (segment (start 108.204 98.552) (end 90.354179 98.552) (width 0.3) (layer "F.Cu") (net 2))
 (segment (start 89.408 95.216097) (end 89.229138 95.394959) (width 0.3) (layer "F.Cu") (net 2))
 (segment (start 107.188 85.852) (end 109.22 87.884) (width 0.3) (layer "F.Cu") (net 2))
 (segment (start 107.188 54.864) (end 107.188 85.852) (width 0.3) (layer "F.Cu") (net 2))
 (segment (start 89.408 97.605821) (end 89.408 95.573821) (width 0.3) (layer "F.Cu") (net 2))
 (segment (start 83.426 52.832) (end 105.156 52.832) (width 0.3) (layer "F.Cu") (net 2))
 (segment (start 79.4 62) (end 78.099 60.699) (width 0.3) (layer "F.Cu") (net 2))
 (segment (start 109.22 87.884) (end 109.22 97.536) (width 0.3) (layer "F.Cu") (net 2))
 (segment (start 90.354179 98.552) (end 89.408 97.605821) (width 0.3) (layer "F.Cu") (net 2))
 (segment (start 105.156 52.832) (end 107.188 54.864) (width 0.3) (layer "F.Cu") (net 2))
 (segment (start 89.408 95.573821) (end 89.229138 95.394959) (width 0.3) (layer "F.Cu") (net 2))
 (segment (start 78.099 58.159) (end 83.426 52.832) (width 0.3) (layer "F.Cu") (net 2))
 (segment (start 78.099 60.699) (end 78.099 58.159) (width 0.3) (layer "F.Cu") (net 2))
 (segment (start 109.22 97.536) (end 108.204 98.552) (width 0.3) (layer "F.Cu") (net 2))
 (segment (start 88.9 89.408) (end 98.482179 89.408) (width 0.5) (layer "B.Cu") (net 15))
 (segment (start 105.664 56.189) (end 104.81 55.335) (width 0.5) (layer "B.Cu") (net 15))
 (segment (start 83.288 95.02) (end 88.9 89.408) (width 0.5) (layer "B.Cu") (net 15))
 (segment (start 104.105089 89.442911) (end 105.664 87.884) (width 0.5) (layer "B.Cu") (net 15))
 (segment (start 79.4 95.02) (end 83.288 95.02) (width 0.5) (layer "B.Cu") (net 15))
 (segment (start 105.664 87.884) (end 105.664 56.189) (width 0.5) (layer "B.Cu") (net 15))
 (segment (start 104.105089 89.442911) (end 104.469138 89.80696) (width 0.5) (layer "B.Cu") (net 15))
 (segment (start 98.482179 89.408) (end 98.517089 89.442911) (width 0.5) (layer "B.Cu") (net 15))
 (segment (start 104.469138 89.80696) (end 104.469138 95.394959) (width 0.5) (layer "B.Cu") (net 15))
 (segment (start 98.517089 89.442911) (end 104.105089 89.442911) (width 0.5) (layer "B.Cu") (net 15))
 (segment (start 88.15 74.7) (end 79.4 74.7) (width 0.3) (layer "B.Cu") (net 7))
 (segment (start 92.11 70.74) (end 92.11 55.335) (width 0.3) (layer "B.Cu") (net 7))
 (segment (start 88.15 74.7) (end 92.11 70.74) (width 0.3) (layer "B.Cu") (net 7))
 (segment (start 79.4 72.16) (end 79.49 72.16) (width 0.3) (layer "F.Cu") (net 6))
 (segment (start 79.84 71.72) (end 88.18 71.72) (width 0.3) (layer "B.Cu") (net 6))
 (segment (start 89.57 70.33) (end 89.57 55.335) (width 0.3) (layer "B.Cu") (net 6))
 (segment (start 88.18 71.72) (end 89.57 70.33) (width 0.3) (layer "B.Cu") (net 6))
 (segment (start 79.4 72.16) (end 79.84 71.72) (width 0.3) (layer "B.Cu") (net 6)))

